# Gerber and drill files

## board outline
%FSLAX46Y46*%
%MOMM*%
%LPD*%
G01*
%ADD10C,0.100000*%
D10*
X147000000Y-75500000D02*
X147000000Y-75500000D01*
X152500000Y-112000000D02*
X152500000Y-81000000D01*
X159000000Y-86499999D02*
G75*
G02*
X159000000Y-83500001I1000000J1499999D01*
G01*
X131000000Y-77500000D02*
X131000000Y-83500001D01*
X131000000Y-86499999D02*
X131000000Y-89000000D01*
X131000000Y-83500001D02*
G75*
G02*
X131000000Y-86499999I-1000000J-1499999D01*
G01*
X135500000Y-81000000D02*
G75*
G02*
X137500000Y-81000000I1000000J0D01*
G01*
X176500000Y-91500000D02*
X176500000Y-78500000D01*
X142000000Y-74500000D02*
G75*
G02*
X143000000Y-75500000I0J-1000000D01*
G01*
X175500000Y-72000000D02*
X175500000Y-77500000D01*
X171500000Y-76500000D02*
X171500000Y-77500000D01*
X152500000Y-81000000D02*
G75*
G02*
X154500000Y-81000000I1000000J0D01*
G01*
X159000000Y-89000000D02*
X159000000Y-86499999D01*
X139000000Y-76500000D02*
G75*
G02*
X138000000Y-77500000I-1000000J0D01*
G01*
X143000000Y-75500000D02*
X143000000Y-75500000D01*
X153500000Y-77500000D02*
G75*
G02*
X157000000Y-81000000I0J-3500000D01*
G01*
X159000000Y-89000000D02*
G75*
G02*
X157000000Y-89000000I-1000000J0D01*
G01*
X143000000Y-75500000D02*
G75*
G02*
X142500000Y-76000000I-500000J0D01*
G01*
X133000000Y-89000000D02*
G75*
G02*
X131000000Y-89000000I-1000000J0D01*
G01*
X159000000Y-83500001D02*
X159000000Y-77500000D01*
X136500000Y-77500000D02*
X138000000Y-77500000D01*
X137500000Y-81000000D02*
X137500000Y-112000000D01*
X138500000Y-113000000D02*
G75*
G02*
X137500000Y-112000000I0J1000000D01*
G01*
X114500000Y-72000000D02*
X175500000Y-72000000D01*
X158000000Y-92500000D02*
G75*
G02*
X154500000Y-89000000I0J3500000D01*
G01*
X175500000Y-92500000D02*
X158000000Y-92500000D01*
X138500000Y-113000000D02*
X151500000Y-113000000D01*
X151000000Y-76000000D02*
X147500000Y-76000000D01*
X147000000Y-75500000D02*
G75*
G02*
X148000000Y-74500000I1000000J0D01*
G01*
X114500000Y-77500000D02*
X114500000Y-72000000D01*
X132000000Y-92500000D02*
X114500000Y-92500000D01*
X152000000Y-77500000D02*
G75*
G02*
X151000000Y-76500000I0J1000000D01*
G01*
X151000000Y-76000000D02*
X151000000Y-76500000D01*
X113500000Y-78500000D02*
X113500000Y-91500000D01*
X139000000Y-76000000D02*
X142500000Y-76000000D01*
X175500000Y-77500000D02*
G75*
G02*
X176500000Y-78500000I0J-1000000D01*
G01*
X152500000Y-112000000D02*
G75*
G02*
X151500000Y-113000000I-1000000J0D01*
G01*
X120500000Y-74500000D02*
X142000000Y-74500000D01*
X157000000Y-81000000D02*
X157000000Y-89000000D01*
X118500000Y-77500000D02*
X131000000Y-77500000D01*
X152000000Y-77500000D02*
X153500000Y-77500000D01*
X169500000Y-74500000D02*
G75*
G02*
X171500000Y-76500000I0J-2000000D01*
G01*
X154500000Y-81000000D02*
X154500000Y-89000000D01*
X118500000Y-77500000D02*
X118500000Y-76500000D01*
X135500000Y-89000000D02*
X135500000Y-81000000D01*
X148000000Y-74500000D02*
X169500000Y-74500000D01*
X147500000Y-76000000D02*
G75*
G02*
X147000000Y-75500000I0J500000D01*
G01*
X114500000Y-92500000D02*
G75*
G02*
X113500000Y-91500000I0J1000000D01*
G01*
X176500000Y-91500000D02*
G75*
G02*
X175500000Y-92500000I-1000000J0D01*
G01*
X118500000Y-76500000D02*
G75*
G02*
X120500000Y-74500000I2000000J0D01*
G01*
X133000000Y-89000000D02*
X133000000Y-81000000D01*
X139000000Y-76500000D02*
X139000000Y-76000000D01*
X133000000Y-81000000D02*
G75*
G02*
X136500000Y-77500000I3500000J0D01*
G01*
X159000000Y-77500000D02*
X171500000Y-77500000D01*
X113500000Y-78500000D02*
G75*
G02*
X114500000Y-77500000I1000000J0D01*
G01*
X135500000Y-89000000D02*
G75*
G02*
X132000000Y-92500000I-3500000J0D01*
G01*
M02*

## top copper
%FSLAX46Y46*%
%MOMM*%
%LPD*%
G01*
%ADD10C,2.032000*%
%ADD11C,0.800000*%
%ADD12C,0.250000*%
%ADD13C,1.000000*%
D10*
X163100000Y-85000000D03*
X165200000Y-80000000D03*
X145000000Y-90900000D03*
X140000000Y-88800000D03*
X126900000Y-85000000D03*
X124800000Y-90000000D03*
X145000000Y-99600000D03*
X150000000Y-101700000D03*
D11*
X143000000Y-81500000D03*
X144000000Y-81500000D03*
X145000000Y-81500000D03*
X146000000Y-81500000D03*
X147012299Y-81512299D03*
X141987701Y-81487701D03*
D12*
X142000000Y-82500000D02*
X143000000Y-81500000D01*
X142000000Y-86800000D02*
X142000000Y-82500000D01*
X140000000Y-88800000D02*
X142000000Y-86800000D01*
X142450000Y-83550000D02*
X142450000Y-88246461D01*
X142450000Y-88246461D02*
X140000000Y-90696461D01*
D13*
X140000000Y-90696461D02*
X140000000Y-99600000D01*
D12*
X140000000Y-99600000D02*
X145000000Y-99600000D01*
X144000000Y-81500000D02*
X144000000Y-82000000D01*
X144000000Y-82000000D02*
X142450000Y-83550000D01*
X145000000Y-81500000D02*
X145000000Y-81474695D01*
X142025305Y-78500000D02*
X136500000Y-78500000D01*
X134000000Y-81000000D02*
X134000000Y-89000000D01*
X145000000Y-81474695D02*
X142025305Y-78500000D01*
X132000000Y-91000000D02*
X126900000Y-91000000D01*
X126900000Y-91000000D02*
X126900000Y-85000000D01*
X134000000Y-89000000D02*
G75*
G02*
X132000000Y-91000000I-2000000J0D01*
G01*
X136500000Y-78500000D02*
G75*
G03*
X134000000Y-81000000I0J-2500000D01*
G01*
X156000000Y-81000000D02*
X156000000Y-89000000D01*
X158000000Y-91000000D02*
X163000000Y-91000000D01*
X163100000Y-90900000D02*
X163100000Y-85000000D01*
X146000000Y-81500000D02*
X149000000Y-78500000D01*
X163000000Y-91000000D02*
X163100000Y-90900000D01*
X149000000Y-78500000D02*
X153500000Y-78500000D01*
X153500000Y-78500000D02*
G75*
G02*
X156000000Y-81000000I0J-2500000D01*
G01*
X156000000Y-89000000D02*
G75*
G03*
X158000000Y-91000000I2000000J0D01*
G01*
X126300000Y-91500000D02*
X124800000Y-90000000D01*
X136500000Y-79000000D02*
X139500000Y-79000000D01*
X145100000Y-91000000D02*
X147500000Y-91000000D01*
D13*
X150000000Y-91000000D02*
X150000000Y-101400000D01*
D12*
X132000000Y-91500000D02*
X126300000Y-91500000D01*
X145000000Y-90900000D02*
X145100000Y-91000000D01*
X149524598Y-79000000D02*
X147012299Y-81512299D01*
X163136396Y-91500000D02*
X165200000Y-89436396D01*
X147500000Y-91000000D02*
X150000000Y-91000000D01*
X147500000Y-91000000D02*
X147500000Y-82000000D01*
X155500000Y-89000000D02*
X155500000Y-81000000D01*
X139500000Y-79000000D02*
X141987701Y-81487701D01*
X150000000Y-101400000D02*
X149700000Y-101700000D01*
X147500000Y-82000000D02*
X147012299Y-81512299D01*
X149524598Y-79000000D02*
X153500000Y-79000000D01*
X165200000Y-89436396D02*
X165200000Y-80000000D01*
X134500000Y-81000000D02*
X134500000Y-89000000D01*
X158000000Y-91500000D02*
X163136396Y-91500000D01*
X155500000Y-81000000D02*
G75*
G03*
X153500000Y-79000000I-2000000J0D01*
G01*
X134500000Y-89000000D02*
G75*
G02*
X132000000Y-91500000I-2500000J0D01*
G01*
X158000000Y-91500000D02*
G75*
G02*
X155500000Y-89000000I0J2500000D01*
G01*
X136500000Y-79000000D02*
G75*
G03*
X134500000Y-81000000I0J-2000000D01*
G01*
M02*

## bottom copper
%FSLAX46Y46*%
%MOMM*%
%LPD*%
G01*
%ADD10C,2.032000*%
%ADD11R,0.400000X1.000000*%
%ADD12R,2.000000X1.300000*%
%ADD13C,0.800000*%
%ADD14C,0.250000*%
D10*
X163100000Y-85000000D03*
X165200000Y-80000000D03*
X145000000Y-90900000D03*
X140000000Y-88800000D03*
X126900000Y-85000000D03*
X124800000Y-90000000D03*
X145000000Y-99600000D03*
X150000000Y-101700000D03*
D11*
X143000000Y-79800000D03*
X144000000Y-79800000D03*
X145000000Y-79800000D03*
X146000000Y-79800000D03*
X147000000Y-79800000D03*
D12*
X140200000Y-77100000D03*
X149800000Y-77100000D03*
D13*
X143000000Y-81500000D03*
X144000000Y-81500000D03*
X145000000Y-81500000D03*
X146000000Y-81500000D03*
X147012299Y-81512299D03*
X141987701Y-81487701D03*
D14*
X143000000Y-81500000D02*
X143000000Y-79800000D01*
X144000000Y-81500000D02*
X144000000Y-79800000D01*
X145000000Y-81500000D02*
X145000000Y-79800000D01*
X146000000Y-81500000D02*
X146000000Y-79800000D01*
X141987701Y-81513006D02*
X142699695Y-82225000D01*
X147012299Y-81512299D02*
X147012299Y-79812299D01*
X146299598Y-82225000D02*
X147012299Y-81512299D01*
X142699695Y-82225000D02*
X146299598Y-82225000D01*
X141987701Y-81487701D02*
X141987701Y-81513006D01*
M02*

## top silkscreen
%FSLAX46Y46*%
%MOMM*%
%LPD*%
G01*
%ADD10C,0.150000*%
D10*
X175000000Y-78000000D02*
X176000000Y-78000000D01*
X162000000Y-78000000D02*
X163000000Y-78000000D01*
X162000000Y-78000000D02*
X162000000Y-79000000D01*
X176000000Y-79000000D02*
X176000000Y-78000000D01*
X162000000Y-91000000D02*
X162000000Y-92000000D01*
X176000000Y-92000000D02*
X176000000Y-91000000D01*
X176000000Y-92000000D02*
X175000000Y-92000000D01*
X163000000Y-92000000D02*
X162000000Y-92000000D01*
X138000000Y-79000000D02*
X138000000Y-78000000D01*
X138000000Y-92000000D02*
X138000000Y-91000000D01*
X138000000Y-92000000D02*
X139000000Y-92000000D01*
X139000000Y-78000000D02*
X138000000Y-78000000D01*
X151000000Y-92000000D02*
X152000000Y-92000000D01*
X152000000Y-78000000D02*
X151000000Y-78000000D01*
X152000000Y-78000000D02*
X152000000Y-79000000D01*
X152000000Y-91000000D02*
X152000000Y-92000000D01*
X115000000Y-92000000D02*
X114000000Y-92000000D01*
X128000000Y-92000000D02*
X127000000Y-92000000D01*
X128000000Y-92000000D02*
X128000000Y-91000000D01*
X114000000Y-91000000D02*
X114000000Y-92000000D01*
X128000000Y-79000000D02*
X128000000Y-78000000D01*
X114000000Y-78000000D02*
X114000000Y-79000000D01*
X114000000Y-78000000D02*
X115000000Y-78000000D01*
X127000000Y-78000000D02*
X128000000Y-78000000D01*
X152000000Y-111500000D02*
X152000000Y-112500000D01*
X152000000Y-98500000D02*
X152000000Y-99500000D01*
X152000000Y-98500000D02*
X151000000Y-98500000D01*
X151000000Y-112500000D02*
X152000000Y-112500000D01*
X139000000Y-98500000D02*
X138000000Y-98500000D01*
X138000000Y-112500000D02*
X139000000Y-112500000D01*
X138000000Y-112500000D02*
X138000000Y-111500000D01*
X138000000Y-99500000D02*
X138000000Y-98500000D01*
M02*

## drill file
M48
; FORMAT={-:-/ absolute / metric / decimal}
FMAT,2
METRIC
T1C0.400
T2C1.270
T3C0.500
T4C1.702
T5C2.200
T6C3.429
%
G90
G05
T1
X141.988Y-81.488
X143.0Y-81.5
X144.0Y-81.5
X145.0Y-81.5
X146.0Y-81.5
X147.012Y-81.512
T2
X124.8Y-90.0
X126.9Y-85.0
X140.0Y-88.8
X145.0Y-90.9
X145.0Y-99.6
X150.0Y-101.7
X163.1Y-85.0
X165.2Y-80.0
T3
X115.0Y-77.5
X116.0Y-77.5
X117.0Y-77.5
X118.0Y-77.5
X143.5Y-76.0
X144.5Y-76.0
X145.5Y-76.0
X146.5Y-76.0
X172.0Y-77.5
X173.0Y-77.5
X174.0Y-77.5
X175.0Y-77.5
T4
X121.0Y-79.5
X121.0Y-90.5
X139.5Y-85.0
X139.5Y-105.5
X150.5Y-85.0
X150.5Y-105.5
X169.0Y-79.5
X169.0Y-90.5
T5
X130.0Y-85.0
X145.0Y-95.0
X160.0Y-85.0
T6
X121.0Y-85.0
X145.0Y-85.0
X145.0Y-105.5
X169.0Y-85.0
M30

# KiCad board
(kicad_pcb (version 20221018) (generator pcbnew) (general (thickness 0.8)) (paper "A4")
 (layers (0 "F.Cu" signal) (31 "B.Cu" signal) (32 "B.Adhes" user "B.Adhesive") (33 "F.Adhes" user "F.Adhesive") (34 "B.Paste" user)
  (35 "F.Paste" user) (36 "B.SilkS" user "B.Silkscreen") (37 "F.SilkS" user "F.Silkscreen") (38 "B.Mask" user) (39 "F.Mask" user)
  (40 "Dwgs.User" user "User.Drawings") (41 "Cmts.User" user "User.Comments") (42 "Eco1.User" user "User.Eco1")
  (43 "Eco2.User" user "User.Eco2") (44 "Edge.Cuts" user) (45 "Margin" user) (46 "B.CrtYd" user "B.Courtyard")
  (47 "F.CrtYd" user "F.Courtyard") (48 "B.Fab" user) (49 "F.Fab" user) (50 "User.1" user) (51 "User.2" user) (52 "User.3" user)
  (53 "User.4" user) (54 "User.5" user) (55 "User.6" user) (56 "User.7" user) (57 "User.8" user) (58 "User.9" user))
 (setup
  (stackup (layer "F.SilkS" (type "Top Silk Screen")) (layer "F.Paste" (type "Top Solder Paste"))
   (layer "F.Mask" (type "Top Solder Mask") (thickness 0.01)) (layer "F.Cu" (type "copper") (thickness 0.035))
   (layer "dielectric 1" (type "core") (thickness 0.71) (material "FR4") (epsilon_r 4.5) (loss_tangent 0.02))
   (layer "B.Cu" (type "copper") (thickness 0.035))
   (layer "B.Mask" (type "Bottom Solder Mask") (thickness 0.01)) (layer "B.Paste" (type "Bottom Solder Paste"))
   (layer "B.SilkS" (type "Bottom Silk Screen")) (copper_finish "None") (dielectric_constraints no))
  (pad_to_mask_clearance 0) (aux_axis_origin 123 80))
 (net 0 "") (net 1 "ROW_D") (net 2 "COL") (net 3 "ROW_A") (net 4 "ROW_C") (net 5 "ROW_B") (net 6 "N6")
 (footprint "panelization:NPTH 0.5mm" (layer "F.Cu") (at 145.5 76)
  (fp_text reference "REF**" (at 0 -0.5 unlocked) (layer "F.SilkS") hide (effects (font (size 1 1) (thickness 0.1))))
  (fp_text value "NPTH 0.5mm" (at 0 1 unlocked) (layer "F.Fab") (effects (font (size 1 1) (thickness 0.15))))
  (pad "" np_thru_hole circle (at 0 0) (size 0.5 0.5) (drill 0.5) (layers "F&B.Cu" "*.Mask")))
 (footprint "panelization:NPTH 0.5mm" (layer "F.Cu") (at 115 77.5)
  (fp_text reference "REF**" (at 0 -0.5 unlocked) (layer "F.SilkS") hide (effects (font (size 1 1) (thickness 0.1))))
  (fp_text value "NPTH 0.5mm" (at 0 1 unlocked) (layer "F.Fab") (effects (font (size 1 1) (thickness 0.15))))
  (pad "" np_thru_hole circle (at 0 0) (size 0.5 0.5) (drill 0.5) (layers "F&B.Cu" "*.Mask")))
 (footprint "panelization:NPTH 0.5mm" (layer "F.Cu") (at 144.5 76)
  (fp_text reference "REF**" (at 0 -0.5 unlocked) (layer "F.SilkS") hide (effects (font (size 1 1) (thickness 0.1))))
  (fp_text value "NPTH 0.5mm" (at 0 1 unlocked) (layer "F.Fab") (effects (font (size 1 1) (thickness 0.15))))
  (pad "" np_thru_hole circle (at 0 0) (size 0.5 0.5) (drill 0.5) (layers "F&B.Cu" "*.Mask")))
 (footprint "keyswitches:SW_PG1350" (layer "F.Cu") (at 169 85 -90)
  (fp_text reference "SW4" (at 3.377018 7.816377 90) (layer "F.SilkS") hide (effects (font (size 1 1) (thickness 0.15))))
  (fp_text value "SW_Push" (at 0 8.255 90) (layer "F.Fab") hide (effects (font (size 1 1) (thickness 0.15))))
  (fp_line (start -7 -6) (end -7 -7) (stroke (width 0.15) (type solid)) (layer "F.SilkS"))
  (fp_line (start -7 7) (end -7 6) (stroke (width 0.15) (type solid)) (layer "F.SilkS"))
  (fp_line (start -7 7) (end -6 7) (stroke (width 0.15) (type solid)) (layer "F.SilkS"))
  (fp_line (start -6 -7) (end -7 -7) (stroke (width 0.15) (type solid)) (layer "F.SilkS"))
  (fp_line (start 6 7) (end 7 7) (stroke (width 0.15) (type solid)) (layer "F.SilkS"))
  (fp_line (start 7 -7) (end 6 -7) (stroke (width 0.15) (type solid)) (layer "F.SilkS"))
  (fp_line (start 7 -7) (end 7 -6) (stroke (width 0.15) (type solid)) (layer "F.SilkS"))
  (fp_line (start 7 6) (end 7 7) (stroke (width 0.15) (type solid)) (layer "F.SilkS"))
  (pad "" np_thru_hole circle (at -5.5 0 270) (size 1.7018 1.7018) (drill 1.7018) (layers "*.Cu" "*.Mask"))
  (pad "" np_thru_hole circle (at 0 0 270) (size 3.429 3.429) (drill 3.429) (layers "*.Cu" "*.Mask"))
  (pad "" np_thru_hole circle (at 5.5 0 270) (size 1.7018 1.7018) (drill 1.7018) (layers "*.Cu" "*.Mask"))
  (pad "1" thru_hole circle (at 0 5.9 270) (size 2.032 2.032) (drill 1.27) (layers "*.Cu" "*.Mask") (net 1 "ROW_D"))
  (pad "2" thru_hole circle (at -5 3.8 270) (size 2.032 2.032) (drill 1.27) (layers "*.Cu" "*.Mask") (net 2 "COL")))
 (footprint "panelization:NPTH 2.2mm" (layer "F.Cu") (at 130 85)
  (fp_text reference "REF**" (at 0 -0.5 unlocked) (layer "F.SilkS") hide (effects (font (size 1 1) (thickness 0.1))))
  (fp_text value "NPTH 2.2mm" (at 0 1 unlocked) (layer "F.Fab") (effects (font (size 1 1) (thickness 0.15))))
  (pad "" np_thru_hole circle (at 0 0) (size 0.0001 0.0001) (drill 2.2) (layers "F&B.Cu")))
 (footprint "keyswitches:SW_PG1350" (layer "F.Cu") (at 145 85)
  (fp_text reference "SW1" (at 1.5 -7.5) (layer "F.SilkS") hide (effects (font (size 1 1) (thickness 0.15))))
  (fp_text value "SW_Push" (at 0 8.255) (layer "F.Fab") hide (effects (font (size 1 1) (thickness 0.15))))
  (fp_line (start -7 -6) (end -7 -7) (stroke (width 0.15) (type solid)) (layer "F.SilkS"))
  (fp_line (start -7 7) (end -7 6) (stroke (width 0.15) (type solid)) (layer "F.SilkS"))
  (fp_line (start -7 7) (end -6 7) (stroke (width 0.15) (type solid)) (layer "F.SilkS"))
  (fp_line (start -6 -7) (end -7 -7) (stroke (width 0.15) (type solid)) (layer "F.SilkS"))
  (fp_line (start 6 7) (end 7 7) (stroke (width 0.15) (type solid)) (layer "F.SilkS"))
  (fp_line (start 7 -7) (end 6 -7) (stroke (width 0.15) (type solid)) (layer "F.SilkS"))
  (fp_line (start 7 -7) (end 7 -6) (stroke (width 0.15) (type solid)) (layer "F.SilkS"))
  (fp_line (start 7 6) (end 7 7) (stroke (width 0.15) (type solid)) (layer "F.SilkS"))
  (pad "" np_thru_hole circle (at -5.5 0) (size 1.7018 1.7018) (drill 1.7018) (layers "*.Cu" "*.Mask"))
  (pad "" np_thru_hole circle (at 0 0) (size 3.429 3.429) (drill 3.429) (layers "*.Cu" "*.Mask"))
  (pad "" np_thru_hole circle (at 5.5 0) (size 1.7018 1.7018) (drill 1.7018) (layers "*.Cu" "*.Mask"))
  (pad "1" thru_hole circle (at 0 5.9) (size 2.032 2.032) (drill 1.27) (layers "*.Cu" "*.Mask") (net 2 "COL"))
  (pad "2" thru_hole circle (at -5 3.8) (size 2.032 2.032) (drill 1.27) (layers "*.Cu" "*.Mask") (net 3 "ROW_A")))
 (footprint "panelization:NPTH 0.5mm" (layer "F.Cu") (at 146.5 76)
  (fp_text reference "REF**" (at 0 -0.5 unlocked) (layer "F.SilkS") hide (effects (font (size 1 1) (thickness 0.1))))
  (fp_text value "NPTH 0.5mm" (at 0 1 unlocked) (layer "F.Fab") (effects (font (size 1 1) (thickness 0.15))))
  (pad "" np_thru_hole circle (at 0 0) (size 0.5 0.5) (drill 0.5) (layers "F&B.Cu" "*.Mask")))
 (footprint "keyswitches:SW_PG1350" (layer "F.Cu") (at 121 85 90)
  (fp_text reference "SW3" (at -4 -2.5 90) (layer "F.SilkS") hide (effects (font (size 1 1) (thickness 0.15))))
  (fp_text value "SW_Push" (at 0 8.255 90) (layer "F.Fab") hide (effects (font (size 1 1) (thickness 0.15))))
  (fp_line (start -7 -6) (end -7 -7) (stroke (width 0.15) (type solid)) (layer "F.SilkS"))
  (fp_line (start -7 7) (end -7 6) (stroke (width 0.15) (type solid)) (layer "F.SilkS"))
  (fp_line (start -7 7) (end -6 7) (stroke (width 0.15) (type solid)) (layer "F.SilkS"))
  (fp_line (start -6 -7) (end -7 -7) (stroke (width 0.15) (type solid)) (layer "F.SilkS"))
  (fp_line (start 6 7) (end 7 7) (stroke (width 0.15) (type solid)) (layer "F.SilkS"))
  (fp_line (start 7 -7) (end 6 -7) (stroke (width 0.15) (type solid)) (layer "F.SilkS"))
  (fp_line (start 7 -7) (end 7 -6) (stroke (width 0.15) (type solid)) (layer "F.SilkS"))
  (fp_line (start 7 6) (end 7 7) (stroke (width 0.15) (type solid)) (layer "F.SilkS"))
  (pad "" np_thru_hole circle (at -5.5 0 90) (size 1.7018 1.7018) (drill 1.7018) (layers "*.Cu" "*.Mask"))
  (pad "" np_thru_hole circle (at 0 0 90) (size 3.429 3.429) (drill 3.429) (layers "*.Cu" "*.Mask"))
  (pad "" np_thru_hole circle (at 5.5 0 90) (size 1.7018 1.7018) (drill 1.7018) (layers "*.Cu" "*.Mask"))
  (pad "1" thru_hole circle (at 0 5.9 90) (size 2.032 2.032) (drill 1.27) (layers "*.Cu" "*.Mask") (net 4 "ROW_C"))
  (pad "2" thru_hole circle (at -5 3.8 90) (size 2.032 2.032) (drill 1.27) (layers "*.Cu" "*.Mask") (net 2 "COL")))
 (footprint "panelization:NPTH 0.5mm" (layer "F.Cu") (at 118 77.5)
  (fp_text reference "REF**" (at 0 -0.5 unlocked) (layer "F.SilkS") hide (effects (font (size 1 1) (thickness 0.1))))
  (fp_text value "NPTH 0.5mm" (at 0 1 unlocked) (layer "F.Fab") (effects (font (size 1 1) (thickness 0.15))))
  (pad "" np_thru_hole circle (at 0 0) (size 0.5 0.5) (drill 0.5) (layers "F&B.Cu" "*.Mask")))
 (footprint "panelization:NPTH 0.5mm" (layer "F.Cu") (at 116 77.5)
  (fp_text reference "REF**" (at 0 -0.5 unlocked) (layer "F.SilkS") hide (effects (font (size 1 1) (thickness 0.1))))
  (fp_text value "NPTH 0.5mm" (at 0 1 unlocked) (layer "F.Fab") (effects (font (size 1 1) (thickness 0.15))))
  (pad "" np_thru_hole circle (at 0 0) (size 0.5 0.5) (drill 0.5) (layers "F&B.Cu" "*.Mask")))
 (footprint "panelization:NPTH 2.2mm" (layer "F.Cu") (at 145 95)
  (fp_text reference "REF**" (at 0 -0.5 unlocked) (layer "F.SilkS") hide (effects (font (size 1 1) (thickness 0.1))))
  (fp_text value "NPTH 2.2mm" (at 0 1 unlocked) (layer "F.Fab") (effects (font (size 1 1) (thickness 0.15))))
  (pad "" np_thru_hole circle (at 0 0) (size 0.0001 0.0001) (drill 2.2) (layers "F&B.Cu")))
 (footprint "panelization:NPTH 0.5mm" (layer "F.Cu") (at 143.5 76)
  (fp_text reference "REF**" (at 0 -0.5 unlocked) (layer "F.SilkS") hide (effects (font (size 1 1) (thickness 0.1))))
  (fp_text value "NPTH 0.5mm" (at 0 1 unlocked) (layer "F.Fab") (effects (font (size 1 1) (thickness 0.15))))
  (pad "" np_thru_hole circle (at 0 0) (size 0.5 0.5) (drill 0.5) (layers "F&B.Cu" "*.Mask")))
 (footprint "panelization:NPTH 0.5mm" (layer "F.Cu") (at 117 77.5)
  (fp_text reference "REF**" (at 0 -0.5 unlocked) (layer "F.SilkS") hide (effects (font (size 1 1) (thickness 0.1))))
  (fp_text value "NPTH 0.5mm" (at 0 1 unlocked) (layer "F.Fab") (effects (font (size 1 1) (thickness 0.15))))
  (pad "" np_thru_hole circle (at 0 0) (size 0.5 0.5) (drill 0.5) (layers "F&B.Cu" "*.Mask")))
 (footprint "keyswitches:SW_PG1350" (layer "F.Cu") (at 145 105.5 180)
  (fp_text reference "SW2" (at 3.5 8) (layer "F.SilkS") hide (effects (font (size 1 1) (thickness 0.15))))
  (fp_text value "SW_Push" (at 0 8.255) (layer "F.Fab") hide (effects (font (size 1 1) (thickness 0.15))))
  (fp_line (start -7 -6) (end -7 -7) (stroke (width 0.15) (type solid)) (layer "F.SilkS"))
  (fp_line (start -7 7) (end -7 6) (stroke (width 0.15) (type solid)) (layer "F.SilkS"))
  (fp_line (start -7 7) (end -6 7) (stroke (width 0.15) (type solid)) (layer "F.SilkS"))
  (fp_line (start -6 -7) (end -7 -7) (stroke (width 0.15) (type solid)) (layer "F.SilkS"))
  (fp_line (start 6 7) (end 7 7) (stroke (width 0.15) (type solid)) (layer "F.SilkS"))
  (fp_line (start 7 -7) (end 6 -7) (stroke (width 0.15) (type solid)) (layer "F.SilkS"))
  (fp_line (start 7 -7) (end 7 -6) (stroke (width 0.15) (type solid)) (layer "F.SilkS"))
  (fp_line (start 7 6) (end 7 7) (stroke (width 0.15) (type solid)) (layer "F.SilkS"))
  (pad "" np_thru_hole circle (at -5.5 0 180) (size 1.7018 1.7018) (drill 1.7018) (layers "*.Cu" "*.Mask"))
  (pad "" np_thru_hole circle (at 0 0 180) (size 3.429 3.429) (drill 3.429) (layers "*.Cu" "*.Mask"))
  (pad "" np_thru_hole circle (at 5.5 0 180) (size 1.7018 1.7018) (drill 1.7018) (layers "*.Cu" "*.Mask"))
  (pad "1" thru_hole circle (at 0 5.9 180) (size 2.032 2.032) (drill 1.27) (layers "*.Cu" "*.Mask") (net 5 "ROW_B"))
  (pad "2" thru_hole circle (at -5 3.8 180) (size 2.032 2.032) (drill 1.27) (layers "*.Cu" "*.Mask") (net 2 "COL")))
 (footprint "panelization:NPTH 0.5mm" (layer "B.Cu") (at 175 77.5 180)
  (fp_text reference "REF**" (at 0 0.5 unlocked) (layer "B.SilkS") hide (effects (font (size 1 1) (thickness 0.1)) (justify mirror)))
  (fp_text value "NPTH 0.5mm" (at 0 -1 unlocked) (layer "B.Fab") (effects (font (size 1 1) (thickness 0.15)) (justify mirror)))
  (pad "" np_thru_hole circle (at 0 0 180) (size 0.5 0.5) (drill 0.5) (layers "F&B.Cu" "*.Mask")))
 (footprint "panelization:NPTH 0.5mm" (layer "B.Cu") (at 174 77.5 180)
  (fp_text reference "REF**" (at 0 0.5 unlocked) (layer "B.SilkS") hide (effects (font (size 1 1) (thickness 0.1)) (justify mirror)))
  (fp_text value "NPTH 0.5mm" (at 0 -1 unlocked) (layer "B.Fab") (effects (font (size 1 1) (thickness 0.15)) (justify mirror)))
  (pad "" np_thru_hole circle (at 0 0 180) (size 0.5 0.5) (drill 0.5) (layers "F&B.Cu" "*.Mask")))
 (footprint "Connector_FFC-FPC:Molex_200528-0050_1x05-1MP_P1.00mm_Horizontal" (layer "B.Cu") (at 145 78.89)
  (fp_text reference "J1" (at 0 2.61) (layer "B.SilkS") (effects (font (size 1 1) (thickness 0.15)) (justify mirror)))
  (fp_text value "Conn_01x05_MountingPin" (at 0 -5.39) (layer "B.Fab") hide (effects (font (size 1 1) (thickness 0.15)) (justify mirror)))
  (pad "1" smd rect (at -2 0.91) (size 0.4 1) (layers "B.Cu" "B.Paste" "B.Mask") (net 3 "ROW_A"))
  (pad "2" smd rect (at -1 0.91) (size 0.4 1) (layers "B.Cu" "B.Paste" "B.Mask") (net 5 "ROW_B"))
  (pad "3" smd rect (at 0 0.91) (size 0.4 1) (layers "B.Cu" "B.Paste" "B.Mask") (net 4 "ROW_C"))
  (pad "4" smd rect (at 1 0.91) (size 0.4 1) (layers "B.Cu" "B.Paste" "B.Mask") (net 1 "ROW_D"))
  (pad "5" smd rect (at 2 0.91) (size 0.4 1) (layers "B.Cu" "B.Paste" "B.Mask") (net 2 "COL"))
  (pad "MP" smd rect (at -4.8 -1.79) (size 2 1.3) (layers "B.Cu" "B.Paste" "B.Mask") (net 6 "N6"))
  (pad "MP" smd rect (at 4.8 -1.79) (size 2 1.3) (layers "B.Cu" "B.Paste" "B.Mask") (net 6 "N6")))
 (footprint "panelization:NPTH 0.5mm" (layer "B.Cu") (at 173 77.5 180)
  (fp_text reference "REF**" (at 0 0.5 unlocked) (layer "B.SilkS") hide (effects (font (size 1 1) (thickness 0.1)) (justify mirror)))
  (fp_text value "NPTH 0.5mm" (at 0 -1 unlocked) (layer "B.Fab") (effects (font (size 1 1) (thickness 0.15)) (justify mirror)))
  (pad "" np_thru_hole circle (at 0 0 180) (size 0.5 0.5) (drill 0.5) (layers "F&B.Cu" "*.Mask")))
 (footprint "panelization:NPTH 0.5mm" (layer "B.Cu") (at 172 77.5 180)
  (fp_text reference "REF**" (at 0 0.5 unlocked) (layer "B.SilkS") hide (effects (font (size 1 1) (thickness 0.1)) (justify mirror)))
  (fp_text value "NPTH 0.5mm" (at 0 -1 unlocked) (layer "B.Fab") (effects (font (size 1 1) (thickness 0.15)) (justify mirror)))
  (pad "" np_thru_hole circle (at 0 0 180) (size 0.5 0.5) (drill 0.5) (layers "F&B.Cu" "*.Mask")))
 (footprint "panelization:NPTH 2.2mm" (layer "B.Cu") (at 160 85 180)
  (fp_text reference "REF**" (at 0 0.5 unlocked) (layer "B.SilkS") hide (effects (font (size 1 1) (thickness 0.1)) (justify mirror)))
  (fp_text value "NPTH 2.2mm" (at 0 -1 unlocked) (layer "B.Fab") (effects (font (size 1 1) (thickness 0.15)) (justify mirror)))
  (pad "" np_thru_hole circle (at 0 0 180) (size 0.0001 0.0001) (drill 2.2) (layers "F&B.Cu")))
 (gr_line (start 147 75.5) (end 147 75.5) (stroke (width 0.1) (type default)) (layer "Edge.Cuts"))
 (gr_line (start 152.5 112) (end 152.5 81) (stroke (width 0.1) (type default)) (layer "Edge.Cuts"))
 (gr_arc (start 159 86.499999) (mid 158.197225 85) (end 159 83.500001) (stroke (width 0.1) (type default)) (layer "Edge.Cuts"))
 (gr_line (start 131 77.5) (end 131 83.500001) (stroke (width 0.1) (type default)) (layer "Edge.Cuts"))
 (gr_line (start 131 86.499999) (end 131 89) (stroke (width 0.1) (type default)) (layer "Edge.Cuts"))
 (gr_arc (start 131 83.500001) (mid 131.802775 85) (end 131 86.499999) (stroke (width 0.1) (type default)) (layer "Edge.Cuts"))
 (gr_arc (start 135.5 81) (mid 136.5 80) (end 137.5 81) (stroke (width 0.1) (type default)) (layer "Edge.Cuts"))
 (gr_line (start 176.5 91.5) (end 176.5 78.5) (stroke (width 0.1) (type default)) (layer "Edge.Cuts"))
 (gr_arc (start 142 74.5) (mid 142.707107 74.792893) (end 143 75.5) (stroke (width 0.1) (type default)) (layer "Edge.Cuts"))
 (gr_line (start 175.5 72) (end 175.5 77.5) (stroke (width 0.1) (type default)) (layer "Edge.Cuts"))
 (gr_line (start 171.5 76.5) (end 171.5 77.5) (stroke (width 0.1) (type default)) (layer "Edge.Cuts"))
 (gr_arc (start 152.5 81) (mid 153.5 80) (end 154.5 81) (stroke (width 0.1) (type default)) (layer "Edge.Cuts"))
 (gr_line (start 159 89) (end 159 86.499999) (stroke (width 0.1) (type default)) (layer "Edge.Cuts"))
 (gr_arc (start 139 76.5) (mid 138.707107 77.207107) (end 138 77.5) (stroke (width 0.1) (type default)) (layer "Edge.Cuts"))
 (gr_line (start 143 75.5) (end 143 75.5) (stroke (width 0.1) (type default)) (layer "Edge.Cuts"))
 (gr_arc (start 153.5 77.5) (mid 155.974874 78.525126) (end 157 81) (stroke (width 0.1) (type default)) (layer "Edge.Cuts"))
 (gr_arc (start 159 89) (mid 158 90) (end 157 89) (stroke (width 0.1) (type default)) (layer "Edge.Cuts"))
 (gr_arc (start 143 75.5) (mid 142.853553 75.853553) (end 142.5 76) (stroke (width 0.1) (type default)) (layer "Edge.Cuts"))
 (gr_arc (start 133 89) (mid 132 90) (end 131 89) (stroke (width 0.1) (type default)) (layer "Edge.Cuts"))
 (gr_line (start 159 83.500001) (end 159 77.5) (stroke (width 0.1) (type default)) (layer "Edge.Cuts"))
 (gr_line (start 136.5 77.5) (end 138 77.5) (stroke (width 0.1) (type default)) (layer "Edge.Cuts"))
 (gr_line (start 137.5 81) (end 137.5 112) (stroke (width 0.1) (type default)) (layer "Edge.Cuts"))
 (gr_arc (start 138.5 113) (mid 137.792893 112.707107) (end 137.5 112) (stroke (width 0.1) (type default)) (layer "Edge.Cuts"))
 (gr_line (start 114.5 72) (end 175.5 72) (stroke (width 0.1) (type default)) (layer "Edge.Cuts"))
 (gr_arc (start 158 92.5) (mid 155.525126 91.474874) (end 154.5 89) (stroke (width 0.1) (type default)) (layer "Edge.Cuts"))
 (gr_line (start 175.5 92.5) (end 158 92.5) (stroke (width 0.1) (type default)) (layer "Edge.Cuts"))
 (gr_line (start 138.5 113) (end 151.5 113) (stroke (width 0.1) (type default)) (layer "Edge.Cuts"))
 (gr_line (start 151 76) (end 147.5 76) (stroke (width 0.1) (type default)) (layer "Edge.Cuts"))
 (gr_arc (start 147 75.5) (mid 147.292893 74.792893) (end 148 74.5) (stroke (width 0.1) (type default)) (layer "Edge.Cuts"))
 (gr_line (start 114.5 77.5) (end 114.5 72) (stroke (width 0.1) (type default)) (layer "Edge.Cuts"))
 (gr_line (start 132 92.5) (end 114.5 92.5) (stroke (width 0.1) (type default)) (layer "Edge.Cuts"))
 (gr_arc (start 152 77.5) (mid 151.292893 77.207107) (end 151 76.5) (stroke (width 0.1) (type default)) (layer "Edge.Cuts"))
 (gr_line (start 151 76) (end 151 76.5) (stroke (width 0.1) (type default)) (layer "Edge.Cuts"))
 (gr_line (start 113.5 78.5) (end 113.5 91.5) (stroke (width 0.1) (type default)) (layer "Edge.Cuts"))
 (gr_line (start 139 76) (end 142.5 76) (stroke (width 0.1) (type default)) (layer "Edge.Cuts"))
 (gr_arc (start 175.5 77.5) (mid 176.207107 77.792893) (end 176.5 78.5) (stroke (width 0.1) (type default)) (layer "Edge.Cuts"))
 (gr_arc (start 152.5 112) (mid 152.207107 112.707107) (end 151.5 113) (stroke (width 0.1) (type default)) (layer "Edge.Cuts"))
 (gr_line (start 120.5 74.5) (end 142 74.5) (stroke (width 0.1) (type default)) (layer "Edge.Cuts"))
 (gr_line (start 157 81) (end 157 89) (stroke (width 0.1) (type default)) (layer "Edge.Cuts"))
 (gr_line (start 118.5 77.5) (end 131 77.5) (stroke (width 0.1) (type default)) (layer "Edge.Cuts"))
 (gr_line (start 152 77.5) (end 153.5 77.5) (stroke (width 0.1) (type default)) (layer "Edge.Cuts"))
 (gr_arc (start 169.5 74.5) (mid 170.914214 75.085786) (end 171.5 76.5) (stroke (width 0.1) (type default)) (layer "Edge.Cuts"))
 (gr_line (start 154.5 81) (end 154.5 89) (stroke (width 0.1) (type default)) (layer "Edge.Cuts"))
 (gr_line (start 118.5 77.5) (end 118.5 76.5) (stroke (width 0.1) (type default)) (layer "Edge.Cuts"))
 (gr_line (start 135.5 89) (end 135.5 81) (stroke (width 0.1) (type default)) (layer "Edge.Cuts"))
 (gr_line (start 148 74.5) (end 169.5 74.5) (stroke (width 0.1) (type default)) (layer "Edge.Cuts"))
 (gr_arc (start 147.5 76) (mid 147.146447 75.853553) (end 147 75.5) (stroke (width 0.1) (type default)) (layer "Edge.Cuts"))
 (gr_arc (start 114.5 92.5) (mid 113.792893 92.207107) (end 113.5 91.5) (stroke (width 0.1) (type default)) (layer "Edge.Cuts"))
 (gr_arc (start 176.5 91.5) (mid 176.207107 92.207107) (end 175.5 92.5) (stroke (width 0.1) (type default)) (layer "Edge.Cuts"))
 (gr_arc (start 118.5 76.5) (mid 119.085786 75.085786) (end 120.5 74.5) (stroke (width 0.1) (type default)) (layer "Edge.Cuts"))
 (gr_line (start 133 89) (end 133 81) (stroke (width 0.1) (type default)) (layer "Edge.Cuts"))
 (gr_line (start 139 76.5) (end 139 76) (stroke (width 0.1) (type default)) (layer "Edge.Cuts"))
 (gr_arc (start 133 81) (mid 134.025126 78.525126) (end 136.5 77.5) (stroke (width 0.1) (type default)) (layer "Edge.Cuts"))
 (gr_line (start 159 77.5) (end 171.5 77.5) (stroke (width 0.1) (type default)) (layer "Edge.Cuts"))
 (gr_arc (start 113.5 78.5) (mid 113.792893 77.792893) (end 114.5 77.5) (stroke (width 0.1) (type default)) (layer "Edge.Cuts"))
 (gr_arc (start 135.5 89) (mid 134.474874 91.474874) (end 132 92.5) (stroke (width 0.1) (type default)) (layer "Edge.Cuts"))
 (segment (start 142 82.5) (end 143 81.5) (width 0.25) (layer "F.Cu") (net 3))
 (segment (start 142 86.8) (end 142 82.5) (width 0.25) (layer "F.Cu") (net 3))
 (segment (start 140 88.8) (end 142 86.8) (width 0.25) (layer "F.Cu") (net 3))
 (via (at 143 81.5) (size 0.8) (drill 0.4) (layers "F.Cu" "B.Cu") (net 3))
 (segment (start 143 81.5) (end 143 79.8) (width 0.25) (layer "B.Cu") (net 3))
 (segment (start 142.45 83.55) (end 142.45 88.246461) (width 0.25) (layer "F.Cu") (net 5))
 (segment (start 142.45 88.246461) (end 140 90.696461) (width 0.25) (layer "F.Cu") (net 5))
 (segment (start 140 90.696461) (end 140 99.6) (width 1) (layer "F.Cu") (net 5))
 (segment (start 140 99.6) (end 145 99.6) (width 0.25) (layer "F.Cu") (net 5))
 (segment (start 144 81.5) (end 144 82) (width 0.25) (layer "F.Cu") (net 5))
 (segment (start 144 82) (end 142.45 83.55) (width 0.25) (layer "F.Cu") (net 5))
 (via (at 144 81.5) (size 0.8) (drill 0.4) (layers "F.Cu" "B.Cu") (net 5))
 (segment (start 144 81.5) (end 144 79.8) (width 0.25) (layer "B.Cu") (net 5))
 (segment (start 145 81.5) (end 145 81.474695) (width 0.25) (layer "F.Cu") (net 4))
 (segment (start 142.025305 78.5) (end 136.5 78.5) (width 0.25) (layer "F.Cu") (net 4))
 (segment (start 134 81) (end 134 89) (width 0.25) (layer "F.Cu") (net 4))
 (segment (start 145 81.474695) (end 142.025305 78.5) (width 0.25) (layer "F.Cu") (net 4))
 (segment (start 132 91) (end 126.9 91) (width 0.25) (layer "F.Cu") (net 4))
 (segment (start 126.9 91) (end 126.9 85) (width 0.25) (layer "F.Cu") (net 4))
 (via (at 145 81.5) (size 0.8) (drill 0.4) (layers "F.Cu" "B.Cu") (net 4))
 (arc (start 134 89) (mid 133.414214 90.414214) (end 132 91) (width 0.25) (layer "F.Cu") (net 4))
 (arc (start 136.5 78.5) (mid 134.732233 79.232233) (end 134 81) (width 0.25) (layer "F.Cu") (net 4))
 (segment (start 145 81.5) (end 145 79.8) (width 0.25) (layer "B.Cu") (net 4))
 (segment (start 156 81) (end 156 89) (width 0.25) (layer "F.Cu") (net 1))
 (segment (start 158 91) (end 163 91) (width 0.25) (layer "F.Cu") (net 1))
 (segment (start 163.1 90.9) (end 163.1 85) (width 0.25) (layer "F.Cu") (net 1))
 (segment (start 146 81.5) (end 149 78.5) (width 0.25) (layer "F.Cu") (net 1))
 (segment (start 163 91) (end 163.1 90.9) (width 0.25) (layer "F.Cu") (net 1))
 (segment (start 149 78.5) (end 153.5 78.5) (width 0.25) (layer "F.Cu") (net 1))
 (via (at 146 81.5) (size 0.8) (drill 0.4) (layers "F.Cu" "B.Cu") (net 1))
 (arc (start 153.5 78.5) (mid 155.267767 79.232233) (end 156 81) (width 0.25) (layer "F.Cu") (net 1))
 (arc (start 156 89) (mid 156.585786 90.414214) (end 158 91) (width 0.25) (layer "F.Cu") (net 1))
 (segment (start 146 81.5) (end 146 79.8) (width 0.25) (layer "B.Cu") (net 1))
 (segment (start 126.3 91.5) (end 124.8 90) (width 0.25) (layer "F.Cu") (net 2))
 (segment (start 136.5 79) (end 139.5 79) (width 0.25) (layer "F.Cu") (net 2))
 (segment (start 145.1 91) (end 147.5 91) (width 0.25) (layer "F.Cu") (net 2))
 (segment (start 150 91) (end 150 101.4) (width 1) (layer "F.Cu") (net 2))
 (segment (start 132 91.5) (end 126.3 91.5) (width 0.25) (layer "F.Cu") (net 2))
 (segment (start 145 90.9) (end 145.1 91) (width 0.25) (layer "F.Cu") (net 2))
 (segment (start 149.524598 79) (end 147.012299 81.512299) (width 0.25) (layer "F.Cu") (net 2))
 (segment (start 163.136396 91.5) (end 165.2 89.436396) (width 0.25) (layer "F.Cu") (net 2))
 (segment (start 147.5 91) (end 150 91) (width 0.25) (layer "F.Cu") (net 2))
 (segment (start 147.5 91) (end 147.5 82) (width 0.25) (layer "F.Cu") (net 2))
 (segment (start 155.5 89) (end 155.5 81) (width 0.25) (layer "F.Cu") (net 2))
 (segment (start 139.5 79) (end 141.987701 81.487701) (width 0.25) (layer "F.Cu") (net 2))
 (segment (start 150 101.4) (end 149.7 101.7) (width 0.25) (layer "F.Cu") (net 2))
 (segment (start 147.5 82) (end 147.012299 81.512299) (width 0.25) (layer "F.Cu") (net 2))
 (segment (start 149.524598 79) (end 153.5 79) (width 0.25) (layer "F.Cu") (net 2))
 (segment (start 165.2 89.436396) (end 165.2 80) (width 0.25) (layer "F.Cu") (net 2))
 (segment (start 134.5 81) (end 134.5 89) (width 0.25) (layer "F.Cu") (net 2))
 (segment (start 158 91.5) (end 163.136396 91.5) (width 0.25) (layer "F.Cu") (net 2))
 (via (at 147.012299 81.512299) (size 0.8) (drill 0.4) (layers "F.Cu" "B.Cu") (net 2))
 (via (at 141.987701 81.487701) (size 0.8) (drill 0.4) (layers "F.Cu" "B.Cu") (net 2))
 (arc (start 155.5 81) (mid 154.914214 79.585786) (end 153.5 79) (width 0.25) (layer "F.Cu") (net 2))
 (arc (start 134.5 89) (mid 133.767767 90.767767) (end 132 91.5) (width 0.25) (layer "F.Cu") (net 2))
 (arc (start 158 91.5) (mid 156.232233 90.767767) (end 155.5 89) (width 0.25) (layer "F.Cu") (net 2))
 (arc (start 136.5 79) (mid 135.085786 79.585786) (end 134.5 81) (width 0.25) (layer "F.Cu") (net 2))
 (segment (start 141.987701 81.513006) (end 142.699695 82.225) (width 0.25) (layer "B.Cu") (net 2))
 (segment (start 147.012299 81.512299) (end 147.012299 79.812299) (width 0.25) (layer "B.Cu") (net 2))
 (segment (start 146.299598 82.225) (end 147.012299 81.512299) (width 0.25) (layer "B.Cu") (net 2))
 (segment (start 142.699695 82.225) (end 146.299598 82.225) (width 0.25) (layer "B.Cu") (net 2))
 (segment (start 141.987701 81.487701) (end 141.987701 81.513006) (width 0.25) (layer "B.Cu") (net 2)))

